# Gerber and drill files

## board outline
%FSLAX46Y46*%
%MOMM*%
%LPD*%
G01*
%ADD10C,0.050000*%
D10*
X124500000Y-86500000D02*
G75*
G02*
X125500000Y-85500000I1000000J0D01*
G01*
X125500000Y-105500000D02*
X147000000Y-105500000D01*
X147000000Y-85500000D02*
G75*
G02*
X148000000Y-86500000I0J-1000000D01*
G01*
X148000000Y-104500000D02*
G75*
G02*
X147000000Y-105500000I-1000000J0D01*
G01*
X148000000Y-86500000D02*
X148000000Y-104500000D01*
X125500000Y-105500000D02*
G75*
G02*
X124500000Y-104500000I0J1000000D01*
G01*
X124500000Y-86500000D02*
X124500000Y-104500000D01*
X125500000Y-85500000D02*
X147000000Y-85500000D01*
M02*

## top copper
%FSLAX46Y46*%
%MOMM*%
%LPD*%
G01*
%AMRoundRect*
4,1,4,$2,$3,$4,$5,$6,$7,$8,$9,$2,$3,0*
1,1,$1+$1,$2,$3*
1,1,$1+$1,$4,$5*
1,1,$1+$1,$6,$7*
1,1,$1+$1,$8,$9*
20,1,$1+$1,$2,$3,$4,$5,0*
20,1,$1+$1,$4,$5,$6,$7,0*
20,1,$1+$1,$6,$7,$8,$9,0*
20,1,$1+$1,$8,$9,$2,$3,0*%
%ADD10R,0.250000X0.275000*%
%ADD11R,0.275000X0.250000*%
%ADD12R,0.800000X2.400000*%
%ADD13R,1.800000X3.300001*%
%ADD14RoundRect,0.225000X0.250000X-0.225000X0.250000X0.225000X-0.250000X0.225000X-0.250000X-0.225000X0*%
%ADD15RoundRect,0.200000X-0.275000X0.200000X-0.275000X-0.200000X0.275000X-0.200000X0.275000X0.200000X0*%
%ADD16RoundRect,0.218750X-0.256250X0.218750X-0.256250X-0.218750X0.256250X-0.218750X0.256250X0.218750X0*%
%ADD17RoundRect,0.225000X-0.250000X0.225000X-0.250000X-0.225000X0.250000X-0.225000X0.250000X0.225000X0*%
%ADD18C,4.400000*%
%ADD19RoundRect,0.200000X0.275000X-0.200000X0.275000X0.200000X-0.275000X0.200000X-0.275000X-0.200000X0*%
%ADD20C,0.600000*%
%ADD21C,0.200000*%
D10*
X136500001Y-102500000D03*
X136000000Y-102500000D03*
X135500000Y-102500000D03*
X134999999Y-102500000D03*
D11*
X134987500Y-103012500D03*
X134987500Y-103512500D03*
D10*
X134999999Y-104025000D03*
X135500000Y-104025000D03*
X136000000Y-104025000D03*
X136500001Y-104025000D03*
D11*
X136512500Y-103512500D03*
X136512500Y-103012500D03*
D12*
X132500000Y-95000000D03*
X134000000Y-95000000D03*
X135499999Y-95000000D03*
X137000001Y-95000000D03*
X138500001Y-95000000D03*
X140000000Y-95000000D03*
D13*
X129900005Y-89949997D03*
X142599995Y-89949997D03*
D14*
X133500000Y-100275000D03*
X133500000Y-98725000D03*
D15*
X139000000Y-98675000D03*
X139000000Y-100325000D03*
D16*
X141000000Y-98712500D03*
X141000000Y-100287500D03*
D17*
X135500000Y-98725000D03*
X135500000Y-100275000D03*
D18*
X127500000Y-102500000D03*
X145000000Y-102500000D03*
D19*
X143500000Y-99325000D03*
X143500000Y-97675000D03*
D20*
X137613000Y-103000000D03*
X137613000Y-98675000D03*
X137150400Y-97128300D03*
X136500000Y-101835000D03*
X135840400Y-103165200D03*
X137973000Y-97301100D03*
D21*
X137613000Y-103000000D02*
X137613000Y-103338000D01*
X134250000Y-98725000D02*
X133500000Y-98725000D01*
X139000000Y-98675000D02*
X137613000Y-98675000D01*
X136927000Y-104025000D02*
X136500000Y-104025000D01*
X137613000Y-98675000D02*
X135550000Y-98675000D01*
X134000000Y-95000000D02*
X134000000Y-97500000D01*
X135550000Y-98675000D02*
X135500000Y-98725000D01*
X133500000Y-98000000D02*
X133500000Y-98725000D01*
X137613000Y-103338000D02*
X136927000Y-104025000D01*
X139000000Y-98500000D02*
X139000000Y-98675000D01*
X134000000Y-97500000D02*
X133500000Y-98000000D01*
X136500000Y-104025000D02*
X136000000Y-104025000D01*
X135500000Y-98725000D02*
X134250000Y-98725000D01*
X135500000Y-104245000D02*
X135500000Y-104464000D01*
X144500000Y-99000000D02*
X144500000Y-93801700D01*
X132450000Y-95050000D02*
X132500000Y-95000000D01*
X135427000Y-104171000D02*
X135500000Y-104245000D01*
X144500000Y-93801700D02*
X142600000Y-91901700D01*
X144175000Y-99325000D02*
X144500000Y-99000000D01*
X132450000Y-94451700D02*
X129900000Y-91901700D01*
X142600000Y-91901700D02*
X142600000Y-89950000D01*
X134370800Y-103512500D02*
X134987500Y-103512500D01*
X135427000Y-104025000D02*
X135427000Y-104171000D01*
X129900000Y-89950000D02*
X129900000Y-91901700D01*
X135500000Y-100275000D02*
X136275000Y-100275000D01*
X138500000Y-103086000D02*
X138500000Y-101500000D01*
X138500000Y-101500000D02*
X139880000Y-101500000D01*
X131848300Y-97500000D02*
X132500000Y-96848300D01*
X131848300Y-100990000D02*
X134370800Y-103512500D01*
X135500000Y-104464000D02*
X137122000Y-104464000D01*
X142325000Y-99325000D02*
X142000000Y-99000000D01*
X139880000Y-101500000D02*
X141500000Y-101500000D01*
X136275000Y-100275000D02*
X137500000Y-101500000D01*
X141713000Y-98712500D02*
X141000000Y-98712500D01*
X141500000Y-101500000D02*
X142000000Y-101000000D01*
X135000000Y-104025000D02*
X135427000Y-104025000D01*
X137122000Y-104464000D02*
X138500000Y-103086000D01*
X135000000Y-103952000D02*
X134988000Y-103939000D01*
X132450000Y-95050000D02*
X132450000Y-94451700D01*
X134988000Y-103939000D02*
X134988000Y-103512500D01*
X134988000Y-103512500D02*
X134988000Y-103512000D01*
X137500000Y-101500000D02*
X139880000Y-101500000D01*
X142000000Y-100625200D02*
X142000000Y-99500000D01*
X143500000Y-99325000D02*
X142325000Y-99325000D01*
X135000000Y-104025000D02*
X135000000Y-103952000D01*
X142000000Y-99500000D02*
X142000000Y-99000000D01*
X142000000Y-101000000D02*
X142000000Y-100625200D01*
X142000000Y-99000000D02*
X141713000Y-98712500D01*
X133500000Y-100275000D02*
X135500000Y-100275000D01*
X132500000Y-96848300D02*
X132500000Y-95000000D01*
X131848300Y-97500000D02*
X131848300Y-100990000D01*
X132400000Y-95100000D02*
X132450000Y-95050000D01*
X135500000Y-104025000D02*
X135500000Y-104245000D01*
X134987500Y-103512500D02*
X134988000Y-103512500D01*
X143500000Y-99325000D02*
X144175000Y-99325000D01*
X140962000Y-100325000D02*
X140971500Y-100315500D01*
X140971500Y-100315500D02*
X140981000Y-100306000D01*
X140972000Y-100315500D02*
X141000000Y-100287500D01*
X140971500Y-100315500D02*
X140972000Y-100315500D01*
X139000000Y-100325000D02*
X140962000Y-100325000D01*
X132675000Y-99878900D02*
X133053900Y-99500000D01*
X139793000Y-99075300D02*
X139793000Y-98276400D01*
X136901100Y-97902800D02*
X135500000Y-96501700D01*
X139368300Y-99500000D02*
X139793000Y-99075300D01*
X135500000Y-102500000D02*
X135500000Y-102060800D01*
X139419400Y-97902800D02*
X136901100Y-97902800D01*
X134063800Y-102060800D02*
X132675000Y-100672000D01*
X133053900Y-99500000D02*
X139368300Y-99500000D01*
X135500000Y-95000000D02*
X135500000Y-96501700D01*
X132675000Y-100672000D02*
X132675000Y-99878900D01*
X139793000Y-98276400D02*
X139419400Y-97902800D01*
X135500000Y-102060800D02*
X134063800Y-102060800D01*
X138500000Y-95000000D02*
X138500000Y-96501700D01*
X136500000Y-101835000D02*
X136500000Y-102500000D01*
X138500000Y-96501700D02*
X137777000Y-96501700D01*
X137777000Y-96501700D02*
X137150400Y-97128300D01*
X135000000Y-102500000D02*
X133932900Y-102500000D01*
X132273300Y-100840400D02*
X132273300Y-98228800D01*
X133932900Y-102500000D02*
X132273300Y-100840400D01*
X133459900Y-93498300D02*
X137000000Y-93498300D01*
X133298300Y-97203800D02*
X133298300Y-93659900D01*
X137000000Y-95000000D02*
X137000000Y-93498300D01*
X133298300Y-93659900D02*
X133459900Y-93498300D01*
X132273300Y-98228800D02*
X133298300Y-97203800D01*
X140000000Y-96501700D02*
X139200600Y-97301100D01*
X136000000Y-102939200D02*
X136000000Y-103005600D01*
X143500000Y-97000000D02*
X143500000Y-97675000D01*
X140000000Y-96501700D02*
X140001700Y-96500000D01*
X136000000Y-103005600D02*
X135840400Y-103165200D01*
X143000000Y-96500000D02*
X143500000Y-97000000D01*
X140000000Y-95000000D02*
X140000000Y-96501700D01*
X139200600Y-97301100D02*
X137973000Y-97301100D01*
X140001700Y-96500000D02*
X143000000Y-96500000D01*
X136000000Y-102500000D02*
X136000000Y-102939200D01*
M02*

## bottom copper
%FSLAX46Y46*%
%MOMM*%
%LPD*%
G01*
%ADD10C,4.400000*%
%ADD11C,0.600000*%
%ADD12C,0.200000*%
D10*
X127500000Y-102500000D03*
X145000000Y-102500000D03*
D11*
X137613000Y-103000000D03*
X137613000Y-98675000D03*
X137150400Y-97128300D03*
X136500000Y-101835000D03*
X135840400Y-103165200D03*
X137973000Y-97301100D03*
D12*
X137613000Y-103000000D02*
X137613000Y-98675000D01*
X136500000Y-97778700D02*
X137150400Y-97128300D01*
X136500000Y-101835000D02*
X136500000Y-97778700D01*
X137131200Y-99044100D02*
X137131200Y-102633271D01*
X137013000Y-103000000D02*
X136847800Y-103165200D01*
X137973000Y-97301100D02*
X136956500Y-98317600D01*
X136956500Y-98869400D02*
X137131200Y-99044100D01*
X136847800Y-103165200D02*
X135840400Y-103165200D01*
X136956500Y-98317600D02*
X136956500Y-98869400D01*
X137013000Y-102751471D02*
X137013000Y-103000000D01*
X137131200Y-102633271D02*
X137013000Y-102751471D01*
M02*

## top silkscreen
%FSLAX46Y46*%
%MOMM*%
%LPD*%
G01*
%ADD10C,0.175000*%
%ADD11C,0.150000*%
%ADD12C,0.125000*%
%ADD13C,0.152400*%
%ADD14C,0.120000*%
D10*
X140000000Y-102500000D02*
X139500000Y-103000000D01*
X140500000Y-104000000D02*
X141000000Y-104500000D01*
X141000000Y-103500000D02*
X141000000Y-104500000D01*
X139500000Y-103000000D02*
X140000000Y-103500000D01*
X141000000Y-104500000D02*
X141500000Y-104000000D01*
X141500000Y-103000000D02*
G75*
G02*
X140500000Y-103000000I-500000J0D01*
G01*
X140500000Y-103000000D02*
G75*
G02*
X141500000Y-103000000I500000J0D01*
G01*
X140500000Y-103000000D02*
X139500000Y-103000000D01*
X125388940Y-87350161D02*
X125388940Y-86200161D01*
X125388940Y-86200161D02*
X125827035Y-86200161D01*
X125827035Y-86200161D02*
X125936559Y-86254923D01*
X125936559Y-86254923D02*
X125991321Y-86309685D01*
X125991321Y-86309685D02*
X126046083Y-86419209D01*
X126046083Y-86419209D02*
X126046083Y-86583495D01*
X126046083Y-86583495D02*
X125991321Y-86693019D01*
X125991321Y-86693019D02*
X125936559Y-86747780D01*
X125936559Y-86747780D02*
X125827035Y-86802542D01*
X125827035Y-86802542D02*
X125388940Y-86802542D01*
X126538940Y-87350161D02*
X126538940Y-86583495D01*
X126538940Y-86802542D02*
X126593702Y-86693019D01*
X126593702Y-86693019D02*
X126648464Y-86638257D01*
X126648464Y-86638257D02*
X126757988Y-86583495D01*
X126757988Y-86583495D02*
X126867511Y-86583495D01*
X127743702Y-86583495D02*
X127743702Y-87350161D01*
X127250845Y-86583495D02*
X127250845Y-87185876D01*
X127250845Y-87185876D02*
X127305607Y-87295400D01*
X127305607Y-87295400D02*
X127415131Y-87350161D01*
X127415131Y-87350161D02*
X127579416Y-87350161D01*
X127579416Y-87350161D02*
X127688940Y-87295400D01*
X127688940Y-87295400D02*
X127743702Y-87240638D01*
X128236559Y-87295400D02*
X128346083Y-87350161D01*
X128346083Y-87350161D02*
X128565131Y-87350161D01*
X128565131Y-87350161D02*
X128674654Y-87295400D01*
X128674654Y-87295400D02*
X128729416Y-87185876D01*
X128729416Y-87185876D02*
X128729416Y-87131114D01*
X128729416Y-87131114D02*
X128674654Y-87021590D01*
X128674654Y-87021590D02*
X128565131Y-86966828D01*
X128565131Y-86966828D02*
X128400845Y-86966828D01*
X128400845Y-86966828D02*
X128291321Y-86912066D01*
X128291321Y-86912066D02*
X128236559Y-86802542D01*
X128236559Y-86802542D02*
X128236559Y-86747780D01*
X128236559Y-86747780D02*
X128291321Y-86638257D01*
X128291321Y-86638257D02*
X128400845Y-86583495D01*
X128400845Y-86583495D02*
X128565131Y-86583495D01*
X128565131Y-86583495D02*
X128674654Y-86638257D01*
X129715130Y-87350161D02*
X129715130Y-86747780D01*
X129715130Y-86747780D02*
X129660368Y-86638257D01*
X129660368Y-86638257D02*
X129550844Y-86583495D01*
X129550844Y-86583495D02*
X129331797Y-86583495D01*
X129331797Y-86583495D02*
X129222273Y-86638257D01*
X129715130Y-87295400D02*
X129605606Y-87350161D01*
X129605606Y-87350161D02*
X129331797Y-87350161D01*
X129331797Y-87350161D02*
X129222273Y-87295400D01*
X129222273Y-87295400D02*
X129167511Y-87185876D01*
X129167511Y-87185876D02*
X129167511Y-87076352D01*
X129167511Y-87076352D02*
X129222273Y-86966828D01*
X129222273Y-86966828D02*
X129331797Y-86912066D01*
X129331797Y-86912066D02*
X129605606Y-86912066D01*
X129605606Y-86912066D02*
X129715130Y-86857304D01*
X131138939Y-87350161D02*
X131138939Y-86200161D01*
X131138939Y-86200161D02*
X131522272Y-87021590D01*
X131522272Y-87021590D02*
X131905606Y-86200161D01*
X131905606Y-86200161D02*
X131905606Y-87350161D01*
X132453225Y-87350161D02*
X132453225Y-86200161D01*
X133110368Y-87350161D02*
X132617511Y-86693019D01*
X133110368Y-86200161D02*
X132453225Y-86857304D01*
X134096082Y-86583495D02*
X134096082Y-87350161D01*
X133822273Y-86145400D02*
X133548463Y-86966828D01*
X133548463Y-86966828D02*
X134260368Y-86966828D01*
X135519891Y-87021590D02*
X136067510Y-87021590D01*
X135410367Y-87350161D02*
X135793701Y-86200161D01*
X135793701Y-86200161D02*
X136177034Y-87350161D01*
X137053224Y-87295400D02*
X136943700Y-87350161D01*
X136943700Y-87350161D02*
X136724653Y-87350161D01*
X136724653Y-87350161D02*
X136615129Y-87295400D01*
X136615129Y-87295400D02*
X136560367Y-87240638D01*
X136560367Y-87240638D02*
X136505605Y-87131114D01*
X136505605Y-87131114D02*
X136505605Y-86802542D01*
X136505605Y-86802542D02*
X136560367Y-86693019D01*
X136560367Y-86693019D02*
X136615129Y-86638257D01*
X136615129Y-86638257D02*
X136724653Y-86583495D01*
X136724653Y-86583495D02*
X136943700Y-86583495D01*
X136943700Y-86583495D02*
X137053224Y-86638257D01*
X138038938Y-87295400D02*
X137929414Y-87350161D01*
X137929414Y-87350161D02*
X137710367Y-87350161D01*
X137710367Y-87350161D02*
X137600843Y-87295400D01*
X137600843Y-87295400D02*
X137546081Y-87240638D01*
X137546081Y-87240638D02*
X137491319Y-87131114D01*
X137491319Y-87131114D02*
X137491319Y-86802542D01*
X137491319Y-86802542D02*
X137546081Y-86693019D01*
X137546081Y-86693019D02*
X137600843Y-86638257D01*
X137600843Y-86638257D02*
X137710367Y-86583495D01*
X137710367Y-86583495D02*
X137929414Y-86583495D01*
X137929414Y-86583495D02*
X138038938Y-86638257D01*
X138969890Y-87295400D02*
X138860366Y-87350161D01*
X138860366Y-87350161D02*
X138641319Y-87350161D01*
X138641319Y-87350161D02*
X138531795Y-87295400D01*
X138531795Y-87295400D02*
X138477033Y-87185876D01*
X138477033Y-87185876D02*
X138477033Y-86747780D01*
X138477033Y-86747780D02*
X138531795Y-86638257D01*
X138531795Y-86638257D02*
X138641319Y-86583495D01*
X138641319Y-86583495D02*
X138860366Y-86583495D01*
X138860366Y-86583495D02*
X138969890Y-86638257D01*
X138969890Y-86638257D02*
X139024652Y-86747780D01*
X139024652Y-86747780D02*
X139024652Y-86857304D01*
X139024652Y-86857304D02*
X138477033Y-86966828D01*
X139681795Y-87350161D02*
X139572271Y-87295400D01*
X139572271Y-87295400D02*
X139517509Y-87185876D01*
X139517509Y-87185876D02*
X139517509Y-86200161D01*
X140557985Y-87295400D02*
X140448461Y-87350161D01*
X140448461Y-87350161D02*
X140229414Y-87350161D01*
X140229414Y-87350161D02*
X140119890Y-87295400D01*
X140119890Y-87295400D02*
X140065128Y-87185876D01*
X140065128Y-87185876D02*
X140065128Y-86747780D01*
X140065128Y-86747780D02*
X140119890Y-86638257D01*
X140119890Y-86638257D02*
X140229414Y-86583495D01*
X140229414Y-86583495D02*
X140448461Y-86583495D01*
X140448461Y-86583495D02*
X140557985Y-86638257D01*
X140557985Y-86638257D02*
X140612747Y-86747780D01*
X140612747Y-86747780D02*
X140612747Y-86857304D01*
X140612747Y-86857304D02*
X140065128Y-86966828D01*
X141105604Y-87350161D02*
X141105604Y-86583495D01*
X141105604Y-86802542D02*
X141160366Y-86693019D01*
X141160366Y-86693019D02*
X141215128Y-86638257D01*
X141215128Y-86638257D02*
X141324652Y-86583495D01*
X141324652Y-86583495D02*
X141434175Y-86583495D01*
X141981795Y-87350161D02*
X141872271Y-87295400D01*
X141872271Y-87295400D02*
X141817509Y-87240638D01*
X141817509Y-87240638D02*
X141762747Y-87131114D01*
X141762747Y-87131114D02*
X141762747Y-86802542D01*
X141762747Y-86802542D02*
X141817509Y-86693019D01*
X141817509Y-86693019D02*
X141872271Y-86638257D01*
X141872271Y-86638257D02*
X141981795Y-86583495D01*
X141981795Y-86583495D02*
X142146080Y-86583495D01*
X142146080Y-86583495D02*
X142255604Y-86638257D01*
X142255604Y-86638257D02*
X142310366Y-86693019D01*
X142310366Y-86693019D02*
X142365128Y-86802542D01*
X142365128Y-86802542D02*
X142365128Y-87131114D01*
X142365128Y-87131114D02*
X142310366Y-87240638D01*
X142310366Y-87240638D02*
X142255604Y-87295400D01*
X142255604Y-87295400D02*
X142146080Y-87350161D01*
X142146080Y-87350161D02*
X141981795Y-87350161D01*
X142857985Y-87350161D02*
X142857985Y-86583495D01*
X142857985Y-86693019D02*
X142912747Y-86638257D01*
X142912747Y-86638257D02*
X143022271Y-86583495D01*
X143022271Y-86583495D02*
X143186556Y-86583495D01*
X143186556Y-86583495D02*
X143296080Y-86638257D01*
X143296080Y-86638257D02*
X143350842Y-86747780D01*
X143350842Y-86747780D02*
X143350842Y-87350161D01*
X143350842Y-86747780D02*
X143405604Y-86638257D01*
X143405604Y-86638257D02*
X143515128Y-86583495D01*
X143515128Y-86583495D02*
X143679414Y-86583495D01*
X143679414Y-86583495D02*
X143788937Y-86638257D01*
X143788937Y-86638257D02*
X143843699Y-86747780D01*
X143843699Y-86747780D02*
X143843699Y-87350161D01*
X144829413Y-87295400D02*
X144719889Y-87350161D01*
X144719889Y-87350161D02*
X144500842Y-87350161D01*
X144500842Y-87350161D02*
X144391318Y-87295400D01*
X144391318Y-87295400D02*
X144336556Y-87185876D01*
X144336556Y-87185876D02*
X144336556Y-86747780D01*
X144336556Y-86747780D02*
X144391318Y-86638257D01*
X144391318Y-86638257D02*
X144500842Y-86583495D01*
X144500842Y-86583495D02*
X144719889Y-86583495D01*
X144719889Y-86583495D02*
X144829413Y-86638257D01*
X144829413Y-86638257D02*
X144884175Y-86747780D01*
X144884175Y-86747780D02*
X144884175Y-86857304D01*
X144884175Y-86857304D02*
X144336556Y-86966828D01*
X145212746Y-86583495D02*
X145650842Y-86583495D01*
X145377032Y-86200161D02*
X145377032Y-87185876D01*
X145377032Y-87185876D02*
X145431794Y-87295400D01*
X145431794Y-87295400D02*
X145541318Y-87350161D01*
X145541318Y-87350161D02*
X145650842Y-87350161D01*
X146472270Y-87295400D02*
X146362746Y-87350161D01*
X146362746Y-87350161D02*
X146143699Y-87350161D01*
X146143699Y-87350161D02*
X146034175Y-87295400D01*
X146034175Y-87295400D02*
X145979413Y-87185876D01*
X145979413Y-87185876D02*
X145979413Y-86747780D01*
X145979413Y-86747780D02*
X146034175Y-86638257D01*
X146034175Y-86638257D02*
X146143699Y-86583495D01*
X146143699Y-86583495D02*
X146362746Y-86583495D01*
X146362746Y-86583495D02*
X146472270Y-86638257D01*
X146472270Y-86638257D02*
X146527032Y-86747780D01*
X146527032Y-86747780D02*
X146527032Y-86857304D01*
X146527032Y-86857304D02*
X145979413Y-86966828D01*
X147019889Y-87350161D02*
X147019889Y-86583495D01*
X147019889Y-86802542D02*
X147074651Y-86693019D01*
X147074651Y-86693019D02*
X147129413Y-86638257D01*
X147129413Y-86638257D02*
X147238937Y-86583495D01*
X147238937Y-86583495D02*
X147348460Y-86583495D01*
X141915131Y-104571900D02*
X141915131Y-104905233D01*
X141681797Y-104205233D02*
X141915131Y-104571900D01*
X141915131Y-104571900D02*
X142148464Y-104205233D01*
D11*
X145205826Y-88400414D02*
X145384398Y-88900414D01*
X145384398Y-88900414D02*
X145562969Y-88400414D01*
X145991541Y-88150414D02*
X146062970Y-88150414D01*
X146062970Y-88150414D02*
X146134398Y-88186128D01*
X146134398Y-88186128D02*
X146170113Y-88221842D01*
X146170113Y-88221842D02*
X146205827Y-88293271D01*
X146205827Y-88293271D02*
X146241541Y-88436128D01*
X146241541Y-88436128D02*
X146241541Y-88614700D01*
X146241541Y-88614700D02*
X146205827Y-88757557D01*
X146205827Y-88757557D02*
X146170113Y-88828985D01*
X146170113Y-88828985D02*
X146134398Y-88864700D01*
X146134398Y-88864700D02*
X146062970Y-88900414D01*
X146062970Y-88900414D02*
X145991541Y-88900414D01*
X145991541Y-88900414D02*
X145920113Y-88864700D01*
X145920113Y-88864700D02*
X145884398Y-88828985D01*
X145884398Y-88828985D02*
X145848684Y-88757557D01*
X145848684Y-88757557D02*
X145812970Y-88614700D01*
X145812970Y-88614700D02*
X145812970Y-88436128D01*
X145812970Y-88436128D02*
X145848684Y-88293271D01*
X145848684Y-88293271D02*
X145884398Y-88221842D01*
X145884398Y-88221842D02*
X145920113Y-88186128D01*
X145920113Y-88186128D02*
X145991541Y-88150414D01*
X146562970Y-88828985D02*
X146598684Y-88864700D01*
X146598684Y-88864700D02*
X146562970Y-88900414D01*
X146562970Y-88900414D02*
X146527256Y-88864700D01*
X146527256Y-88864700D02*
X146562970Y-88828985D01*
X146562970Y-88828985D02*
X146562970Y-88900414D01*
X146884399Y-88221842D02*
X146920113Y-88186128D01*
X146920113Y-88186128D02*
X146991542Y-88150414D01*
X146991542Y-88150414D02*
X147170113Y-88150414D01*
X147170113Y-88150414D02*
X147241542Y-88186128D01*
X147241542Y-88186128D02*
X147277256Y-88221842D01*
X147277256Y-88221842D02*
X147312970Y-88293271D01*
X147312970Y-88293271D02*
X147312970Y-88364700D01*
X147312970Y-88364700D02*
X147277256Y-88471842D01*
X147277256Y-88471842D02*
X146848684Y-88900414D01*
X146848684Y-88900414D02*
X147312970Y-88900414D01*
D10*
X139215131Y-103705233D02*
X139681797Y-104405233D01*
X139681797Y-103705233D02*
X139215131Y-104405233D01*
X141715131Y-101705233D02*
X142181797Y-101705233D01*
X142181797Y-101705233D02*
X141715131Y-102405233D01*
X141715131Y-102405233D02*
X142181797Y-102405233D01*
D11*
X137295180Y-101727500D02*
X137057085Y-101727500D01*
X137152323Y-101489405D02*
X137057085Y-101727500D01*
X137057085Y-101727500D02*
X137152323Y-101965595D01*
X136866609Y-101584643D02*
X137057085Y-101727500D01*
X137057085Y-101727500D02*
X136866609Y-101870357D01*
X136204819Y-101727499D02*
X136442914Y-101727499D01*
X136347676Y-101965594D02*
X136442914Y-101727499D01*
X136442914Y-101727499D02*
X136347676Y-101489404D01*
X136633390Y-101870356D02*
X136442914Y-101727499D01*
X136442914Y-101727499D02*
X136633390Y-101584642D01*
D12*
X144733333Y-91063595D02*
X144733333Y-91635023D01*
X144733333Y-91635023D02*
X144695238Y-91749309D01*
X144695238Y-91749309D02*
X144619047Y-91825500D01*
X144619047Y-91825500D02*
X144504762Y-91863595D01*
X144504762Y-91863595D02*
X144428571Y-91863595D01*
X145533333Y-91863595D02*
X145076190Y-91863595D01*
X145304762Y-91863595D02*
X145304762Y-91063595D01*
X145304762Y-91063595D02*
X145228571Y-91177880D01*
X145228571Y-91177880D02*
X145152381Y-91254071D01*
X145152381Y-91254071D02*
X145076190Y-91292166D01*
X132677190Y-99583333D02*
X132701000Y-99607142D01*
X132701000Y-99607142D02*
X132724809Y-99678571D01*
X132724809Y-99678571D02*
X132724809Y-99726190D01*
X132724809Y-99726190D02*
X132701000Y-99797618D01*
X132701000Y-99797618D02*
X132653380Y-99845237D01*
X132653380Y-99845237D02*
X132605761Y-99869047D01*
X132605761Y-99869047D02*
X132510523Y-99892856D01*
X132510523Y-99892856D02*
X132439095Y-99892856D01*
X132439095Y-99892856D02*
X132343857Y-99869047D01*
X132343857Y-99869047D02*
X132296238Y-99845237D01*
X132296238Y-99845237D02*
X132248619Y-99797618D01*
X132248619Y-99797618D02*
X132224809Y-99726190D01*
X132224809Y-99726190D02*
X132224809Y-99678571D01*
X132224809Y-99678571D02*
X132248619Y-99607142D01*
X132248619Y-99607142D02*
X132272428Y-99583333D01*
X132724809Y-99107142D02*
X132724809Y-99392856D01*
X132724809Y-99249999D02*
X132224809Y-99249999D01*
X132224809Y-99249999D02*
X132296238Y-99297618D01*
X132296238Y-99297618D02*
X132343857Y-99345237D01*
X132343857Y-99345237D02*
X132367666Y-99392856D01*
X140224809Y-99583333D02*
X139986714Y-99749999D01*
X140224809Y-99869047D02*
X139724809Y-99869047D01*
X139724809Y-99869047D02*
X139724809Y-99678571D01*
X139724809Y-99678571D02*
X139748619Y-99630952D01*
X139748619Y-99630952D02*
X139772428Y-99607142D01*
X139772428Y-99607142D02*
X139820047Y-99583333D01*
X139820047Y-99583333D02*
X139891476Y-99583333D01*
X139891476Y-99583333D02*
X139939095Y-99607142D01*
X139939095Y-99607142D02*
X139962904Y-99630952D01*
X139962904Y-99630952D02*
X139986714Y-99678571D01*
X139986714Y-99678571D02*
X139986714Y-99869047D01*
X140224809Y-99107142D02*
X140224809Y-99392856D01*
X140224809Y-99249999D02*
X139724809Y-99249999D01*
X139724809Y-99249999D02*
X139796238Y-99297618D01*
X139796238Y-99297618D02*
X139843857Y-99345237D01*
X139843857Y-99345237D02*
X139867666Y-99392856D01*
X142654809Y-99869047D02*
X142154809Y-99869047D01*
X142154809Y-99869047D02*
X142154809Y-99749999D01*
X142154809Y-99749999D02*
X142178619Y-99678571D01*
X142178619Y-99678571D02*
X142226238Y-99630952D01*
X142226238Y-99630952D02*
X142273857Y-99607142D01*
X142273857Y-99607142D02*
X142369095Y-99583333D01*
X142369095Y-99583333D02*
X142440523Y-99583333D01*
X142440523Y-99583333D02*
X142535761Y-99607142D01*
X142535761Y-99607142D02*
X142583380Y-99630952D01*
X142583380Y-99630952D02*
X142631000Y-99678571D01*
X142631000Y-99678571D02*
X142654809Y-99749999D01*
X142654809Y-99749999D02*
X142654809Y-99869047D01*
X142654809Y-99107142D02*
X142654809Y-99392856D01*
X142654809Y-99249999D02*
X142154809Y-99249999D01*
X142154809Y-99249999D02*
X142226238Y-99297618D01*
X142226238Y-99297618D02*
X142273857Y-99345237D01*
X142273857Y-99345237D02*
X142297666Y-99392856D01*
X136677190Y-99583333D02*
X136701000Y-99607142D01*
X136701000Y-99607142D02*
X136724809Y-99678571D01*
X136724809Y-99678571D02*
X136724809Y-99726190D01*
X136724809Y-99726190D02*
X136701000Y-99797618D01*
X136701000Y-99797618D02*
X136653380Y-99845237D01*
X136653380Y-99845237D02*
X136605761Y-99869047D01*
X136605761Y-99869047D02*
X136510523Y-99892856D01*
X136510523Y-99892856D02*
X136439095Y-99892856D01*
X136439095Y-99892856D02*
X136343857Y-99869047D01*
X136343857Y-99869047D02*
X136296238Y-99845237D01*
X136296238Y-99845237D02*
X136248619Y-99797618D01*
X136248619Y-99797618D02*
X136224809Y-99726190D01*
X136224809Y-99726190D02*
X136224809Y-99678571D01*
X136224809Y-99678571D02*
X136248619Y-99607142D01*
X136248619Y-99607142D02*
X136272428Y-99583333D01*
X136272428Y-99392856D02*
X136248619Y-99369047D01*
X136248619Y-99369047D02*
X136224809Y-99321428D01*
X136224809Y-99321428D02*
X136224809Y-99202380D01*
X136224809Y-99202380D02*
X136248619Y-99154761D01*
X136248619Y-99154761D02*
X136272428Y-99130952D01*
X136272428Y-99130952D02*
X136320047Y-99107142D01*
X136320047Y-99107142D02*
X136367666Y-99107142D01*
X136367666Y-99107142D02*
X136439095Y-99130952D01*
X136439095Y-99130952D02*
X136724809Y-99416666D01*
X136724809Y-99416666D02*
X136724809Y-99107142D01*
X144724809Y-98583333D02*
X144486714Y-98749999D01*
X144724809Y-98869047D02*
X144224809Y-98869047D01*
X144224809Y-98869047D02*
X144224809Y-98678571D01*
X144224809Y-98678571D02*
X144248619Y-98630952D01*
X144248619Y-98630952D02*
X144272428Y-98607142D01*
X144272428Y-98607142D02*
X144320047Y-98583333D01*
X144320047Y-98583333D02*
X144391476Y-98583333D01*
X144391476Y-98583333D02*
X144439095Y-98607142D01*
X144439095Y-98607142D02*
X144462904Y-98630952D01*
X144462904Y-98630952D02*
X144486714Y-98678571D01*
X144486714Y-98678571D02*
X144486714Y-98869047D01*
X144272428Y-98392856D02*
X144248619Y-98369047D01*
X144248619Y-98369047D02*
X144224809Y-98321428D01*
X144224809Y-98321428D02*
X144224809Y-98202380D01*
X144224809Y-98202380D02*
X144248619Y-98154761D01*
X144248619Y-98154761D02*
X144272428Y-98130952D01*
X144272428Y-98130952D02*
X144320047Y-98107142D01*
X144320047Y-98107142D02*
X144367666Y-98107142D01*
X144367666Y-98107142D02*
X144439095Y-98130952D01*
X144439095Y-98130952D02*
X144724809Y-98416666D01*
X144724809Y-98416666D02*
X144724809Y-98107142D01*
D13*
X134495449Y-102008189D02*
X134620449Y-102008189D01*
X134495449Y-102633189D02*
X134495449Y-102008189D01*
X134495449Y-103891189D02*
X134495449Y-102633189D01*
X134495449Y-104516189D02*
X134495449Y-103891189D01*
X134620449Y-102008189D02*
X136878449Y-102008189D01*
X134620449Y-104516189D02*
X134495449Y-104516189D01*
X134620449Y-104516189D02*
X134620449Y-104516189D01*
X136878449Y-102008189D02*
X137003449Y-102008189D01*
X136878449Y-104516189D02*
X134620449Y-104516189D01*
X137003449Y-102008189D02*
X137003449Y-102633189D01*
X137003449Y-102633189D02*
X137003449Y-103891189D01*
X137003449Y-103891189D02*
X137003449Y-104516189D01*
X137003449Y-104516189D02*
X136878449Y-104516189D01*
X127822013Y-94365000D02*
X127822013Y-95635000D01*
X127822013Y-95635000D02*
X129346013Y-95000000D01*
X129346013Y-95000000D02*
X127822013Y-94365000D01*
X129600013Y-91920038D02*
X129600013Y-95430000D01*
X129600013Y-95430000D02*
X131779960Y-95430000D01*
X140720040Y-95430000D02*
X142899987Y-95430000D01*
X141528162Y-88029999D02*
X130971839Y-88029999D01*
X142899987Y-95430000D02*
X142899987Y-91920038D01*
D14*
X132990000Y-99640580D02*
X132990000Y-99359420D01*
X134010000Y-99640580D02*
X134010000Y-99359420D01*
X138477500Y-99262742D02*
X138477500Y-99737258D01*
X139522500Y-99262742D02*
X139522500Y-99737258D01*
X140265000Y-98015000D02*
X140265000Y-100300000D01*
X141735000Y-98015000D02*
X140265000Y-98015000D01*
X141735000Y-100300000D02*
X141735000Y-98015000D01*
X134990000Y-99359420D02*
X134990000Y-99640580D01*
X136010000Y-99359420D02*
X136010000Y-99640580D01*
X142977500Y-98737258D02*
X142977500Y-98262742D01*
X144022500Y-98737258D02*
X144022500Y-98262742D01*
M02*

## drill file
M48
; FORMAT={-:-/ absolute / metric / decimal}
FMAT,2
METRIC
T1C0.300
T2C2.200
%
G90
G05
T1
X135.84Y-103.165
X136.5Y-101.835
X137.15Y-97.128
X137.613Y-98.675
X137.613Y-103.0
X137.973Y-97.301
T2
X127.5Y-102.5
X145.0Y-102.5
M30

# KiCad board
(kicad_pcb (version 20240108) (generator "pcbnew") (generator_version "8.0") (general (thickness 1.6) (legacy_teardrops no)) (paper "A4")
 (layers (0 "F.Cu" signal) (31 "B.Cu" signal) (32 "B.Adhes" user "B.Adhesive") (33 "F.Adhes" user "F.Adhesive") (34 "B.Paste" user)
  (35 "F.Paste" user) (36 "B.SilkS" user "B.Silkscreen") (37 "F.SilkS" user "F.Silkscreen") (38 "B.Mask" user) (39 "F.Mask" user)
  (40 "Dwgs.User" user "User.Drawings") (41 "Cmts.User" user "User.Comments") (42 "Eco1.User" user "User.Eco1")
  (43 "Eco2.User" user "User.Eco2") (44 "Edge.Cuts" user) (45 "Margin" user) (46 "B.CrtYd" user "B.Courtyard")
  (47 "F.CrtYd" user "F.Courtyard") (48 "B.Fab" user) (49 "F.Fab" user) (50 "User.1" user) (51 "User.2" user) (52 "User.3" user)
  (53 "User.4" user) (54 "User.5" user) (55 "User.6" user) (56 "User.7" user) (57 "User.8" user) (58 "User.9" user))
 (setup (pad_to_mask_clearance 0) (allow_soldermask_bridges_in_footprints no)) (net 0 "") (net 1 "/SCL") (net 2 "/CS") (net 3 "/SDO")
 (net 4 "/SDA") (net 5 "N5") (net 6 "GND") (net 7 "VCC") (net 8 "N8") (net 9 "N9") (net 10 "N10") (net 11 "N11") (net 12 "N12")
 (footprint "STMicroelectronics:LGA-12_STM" (layer "F.Cu") (at 135.75 103.2625 -90)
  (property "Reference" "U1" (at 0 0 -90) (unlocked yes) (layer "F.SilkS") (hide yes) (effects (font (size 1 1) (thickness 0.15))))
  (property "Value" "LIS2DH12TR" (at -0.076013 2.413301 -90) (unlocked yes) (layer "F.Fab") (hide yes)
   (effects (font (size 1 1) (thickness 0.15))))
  (fp_line (start -1.254311 1.254551) (end -1.254311 1.129551) (stroke (width 0.1524) (type solid)) (layer "F.SilkS"))
  (fp_line (start -0.629311 1.254551) (end -1.254311 1.254551) (stroke (width 0.1524) (type solid)) (layer "F.SilkS"))
  (fp_line (start 0.628689 1.254551) (end -0.629311 1.254551) (stroke (width 0.1524) (type solid)) (layer "F.SilkS"))
  (fp_line (start 1.253689 1.254551) (end 0.628689 1.254551) (stroke (width 0.1524) (type solid)) (layer "F.SilkS"))
  (fp_line (start -1.254311 1.129551) (end -1.254311 -1.128449) (stroke (width 0.1524) (type solid)) (layer "F.SilkS"))
  (fp_line (start 1.253689 1.129551) (end 1.253689 1.254551) (stroke (width 0.1524) (type solid)) (layer "F.SilkS"))
  (fp_line (start 1.253689 1.129551) (end 1.253689 1.129551) (stroke (width 0.1524) (type solid)) (layer "F.SilkS"))
  (fp_line (start -1.254311 -1.128449) (end -1.254311 -1.253449) (stroke (width 0.1524) (type solid)) (layer "F.SilkS"))
  (fp_line (start 1.253689 -1.128449) (end 1.253689 1.129551) (stroke (width 0.1524) (type solid)) (layer "F.SilkS"))
  (fp_line (start -1.254311 -1.253449) (end -0.629311 -1.253449) (stroke (width 0.1524) (type solid)) (layer "F.SilkS"))
  (fp_line (start -0.629311 -1.253449) (end 0.628689 -1.253449) (stroke (width 0.1524) (type solid)) (layer "F.SilkS"))
  (fp_line (start 0.628689 -1.253449) (end 1.253689 -1.253449) (stroke (width 0.1524) (type solid)) (layer "F.SilkS"))
  (fp_line (start 1.253689 -1.253449) (end 1.253689 -1.128449) (stroke (width 0.1524) (type solid)) (layer "F.SilkS"))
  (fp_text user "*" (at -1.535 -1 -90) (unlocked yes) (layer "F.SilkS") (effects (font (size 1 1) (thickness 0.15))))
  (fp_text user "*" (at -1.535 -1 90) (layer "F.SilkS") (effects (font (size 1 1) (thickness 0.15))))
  (pad "1" smd rect (at -0.7625 -0.750001) (size 0.25 0.275) (layers "F.Cu" "F.Paste" "F.Mask") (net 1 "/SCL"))
  (pad "2" smd rect (at -0.7625 -0.25) (size 0.25 0.275) (layers "F.Cu" "F.Paste" "F.Mask") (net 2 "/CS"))
  (pad "3" smd rect (at -0.7625 0.25) (size 0.25 0.275) (layers "F.Cu" "F.Paste" "F.Mask") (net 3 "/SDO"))
  (pad "4" smd rect (at -0.7625 0.750001) (size 0.25 0.275) (layers "F.Cu" "F.Paste" "F.Mask") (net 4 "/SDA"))
  (pad "5" smd rect (at -0.25 0.7625 270) (size 0.25 0.275) (layers "F.Cu" "F.Paste" "F.Mask") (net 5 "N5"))
  (pad "6" smd rect (at 0.25 0.7625 270) (size 0.25 0.275) (layers "F.Cu" "F.Paste" "F.Mask") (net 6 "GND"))
  (pad "7" smd rect (at 0.7625 0.750001) (size 0.25 0.275) (layers "F.Cu" "F.Paste" "F.Mask") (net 6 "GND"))
  (pad "8" smd rect (at 0.7625 0.25) (size 0.25 0.275) (layers "F.Cu" "F.Paste" "F.Mask") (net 6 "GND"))
  (pad "9" smd rect (at 0.7625 -0.25) (size 0.25 0.275) (layers "F.Cu" "F.Paste" "F.Mask") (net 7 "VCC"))
  (pad "10" smd rect (at 0.7625 -0.750001) (size 0.25 0.275) (layers "F.Cu" "F.Paste" "F.Mask") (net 7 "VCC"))
  (pad "11" smd rect (at 0.25 -0.7625 270) (size 0.25 0.275) (layers "F.Cu" "F.Paste" "F.Mask") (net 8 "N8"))
  (pad "12" smd rect (at -0.25 -0.7625 270) (size 0.25 0.275) (layers "F.Cu" "F.Paste" "F.Mask") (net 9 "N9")))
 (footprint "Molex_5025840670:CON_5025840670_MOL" (layer "F.Cu") (at 132.5 95)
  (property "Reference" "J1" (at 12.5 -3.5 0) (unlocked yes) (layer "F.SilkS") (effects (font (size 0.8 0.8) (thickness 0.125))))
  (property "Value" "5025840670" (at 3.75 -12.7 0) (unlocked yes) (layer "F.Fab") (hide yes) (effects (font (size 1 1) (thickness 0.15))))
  (fp_line (start -4.677987 -0.635) (end -4.677987 0.635) (stroke (width 0.1524) (type solid)) (layer "F.SilkS"))
  (fp_line (start -4.677987 0.635) (end -3.153987 0) (stroke (width 0.1524) (type solid)) (layer "F.SilkS"))
  (fp_line (start -3.153987 0) (end -4.677987 -0.635) (stroke (width 0.1524) (type solid)) (layer "F.SilkS"))
  (fp_line (start -2.899987 -3.079962) (end -2.899987 0.43) (stroke (width 0.1524) (type solid)) (layer "F.SilkS"))
  (fp_line (start -2.899987 0.43) (end -0.72004 0.43) (stroke (width 0.1524) (type solid)) (layer "F.SilkS"))
  (fp_line (start 8.22004 0.43) (end 10.399987 0.43) (stroke (width 0.1524) (type solid)) (layer "F.SilkS"))
  (fp_line (start 9.028162 -6.970001) (end -1.528161 -6.970001) (stroke (width 0.1524) (type solid)) (layer "F.SilkS"))
  (fp_line (start 10.399987 0.43) (end 10.399987 -3.079962) (stroke (width 0.1524) (type solid)) (layer "F.SilkS"))
  (pad "1" smd rect (at 0 0) (size 0.8 2.4) (layers "F.Cu" "F.Paste" "F.Mask") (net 6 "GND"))
  (pad "2" smd rect (at 1.5 0) (size 0.8 2.4) (layers "F.Cu" "F.Paste" "F.Mask") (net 7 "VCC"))
  (pad "3" smd rect (at 2.999999 0) (size 0.8 2.4) (layers "F.Cu" "F.Paste" "F.Mask") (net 3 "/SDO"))
  (pad "4" smd rect (at 4.500001 0) (size 0.8 2.4) (layers "F.Cu" "F.Paste" "F.Mask") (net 4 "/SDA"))
  (pad "5" smd rect (at 6.000001 0) (size 0.8 2.4) (layers "F.Cu" "F.Paste" "F.Mask") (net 1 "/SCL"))
  (pad "6" smd rect (at 7.5 0) (size 0.8 2.4) (layers "F.Cu" "F.Paste" "F.Mask") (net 2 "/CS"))
  (pad "7" smd rect (at -2.599995 -5.050003) (size 1.8 3.300001) (layers "F.Cu" "F.Paste" "F.Mask") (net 6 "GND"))
  (pad "8" smd rect (at 10.099995 -5.050003) (size 1.8 3.300001) (layers "F.Cu" "F.Paste" "F.Mask") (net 6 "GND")))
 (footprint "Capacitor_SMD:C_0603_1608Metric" (layer "F.Cu") (at 133.5 99.5 90)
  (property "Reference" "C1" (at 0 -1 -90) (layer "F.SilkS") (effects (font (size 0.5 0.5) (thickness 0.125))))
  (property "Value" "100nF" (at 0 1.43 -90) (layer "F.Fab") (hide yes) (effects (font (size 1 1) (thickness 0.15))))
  (fp_line (start -0.14058 -0.51) (end 0.14058 -0.51) (stroke (width 0.12) (type solid)) (layer "F.SilkS"))
  (fp_line (start -0.14058 0.51) (end 0.14058 0.51) (stroke (width 0.12) (type solid)) (layer "F.SilkS"))
  (pad "1" smd roundrect (at -0.775 0 90) (size 0.9 0.95) (layers "F.Cu" "F.Paste" "F.Mask") (roundrect_rratio 0.25) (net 6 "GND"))
  (pad "2" smd roundrect (at 0.775 0 90) (size 0.9 0.95) (layers "F.Cu" "F.Paste" "F.Mask") (roundrect_rratio 0.25) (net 7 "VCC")))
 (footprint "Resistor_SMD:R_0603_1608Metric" (layer "F.Cu") (at 139 99.5 -90)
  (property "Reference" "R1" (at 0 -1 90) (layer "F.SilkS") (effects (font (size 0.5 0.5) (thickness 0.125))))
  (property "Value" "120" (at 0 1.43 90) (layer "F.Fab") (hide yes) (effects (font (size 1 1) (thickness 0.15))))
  (fp_line (start -0.237258 0.5225) (end 0.237258 0.5225) (stroke (width 0.12) (type solid)) (layer "F.SilkS"))
  (fp_line (start -0.237258 -0.5225) (end 0.237258 -0.5225) (stroke (width 0.12) (type solid)) (layer "F.SilkS"))
  (pad "1" smd roundrect (at -0.825 0 270) (size 0.8 0.95) (layers "F.Cu" "F.Paste" "F.Mask") (roundrect_rratio 0.25) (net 7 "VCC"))
  (pad "2" smd roundrect (at 0.825 0 270) (size 0.8 0.95) (layers "F.Cu" "F.Paste" "F.Mask") (roundrect_rratio 0.25) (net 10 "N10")))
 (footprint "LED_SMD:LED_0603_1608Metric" (layer "F.Cu") (at 141 99.5 -90)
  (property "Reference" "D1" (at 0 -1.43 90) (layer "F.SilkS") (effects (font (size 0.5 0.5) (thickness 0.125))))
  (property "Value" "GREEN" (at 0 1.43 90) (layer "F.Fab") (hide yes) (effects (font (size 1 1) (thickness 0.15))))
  (fp_line (start -1.485 0.735) (end 0.8 0.735) (stroke (width 0.12) (type solid)) (layer "F.SilkS"))
  (fp_line (start -1.485 -0.735) (end -1.485 0.735) (stroke (width 0.12) (type solid)) (layer "F.SilkS"))
  (fp_line (start 0.8 -0.735) (end -1.485 -0.735) (stroke (width 0.12) (type solid)) (layer "F.SilkS"))
  (pad "1" smd roundrect (at -0.7875 0 270) (size 0.875 0.95) (layers "F.Cu" "F.Paste" "F.Mask") (roundrect_rratio 0.25) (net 6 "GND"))
  (pad "2" smd roundrect (at 0.7875 0 270) (size 0.875 0.95) (layers "F.Cu" "F.Paste" "F.Mask") (roundrect_rratio 0.25) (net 10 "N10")))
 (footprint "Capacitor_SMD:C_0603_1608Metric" (layer "F.Cu") (at 135.5 99.5 -90)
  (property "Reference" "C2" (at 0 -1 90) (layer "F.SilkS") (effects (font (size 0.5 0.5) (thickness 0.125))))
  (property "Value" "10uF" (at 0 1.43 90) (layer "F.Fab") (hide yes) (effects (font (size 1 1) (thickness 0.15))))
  (fp_line (start -0.14058 0.51) (end 0.14058 0.51) (stroke (width 0.12) (type solid)) (layer "F.SilkS"))
  (fp_line (start -0.14058 -0.51) (end 0.14058 -0.51) (stroke (width 0.12) (type solid)) (layer "F.SilkS"))
  (pad "1" smd roundrect (at -0.775 0 270) (size 0.9 0.95) (layers "F.Cu" "F.Paste" "F.Mask") (roundrect_rratio 0.25) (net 7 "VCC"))
  (pad "2" smd roundrect (at 0.775 0 270) (size 0.9 0.95) (layers "F.Cu" "F.Paste" "F.Mask") (roundrect_rratio 0.25) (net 6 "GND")))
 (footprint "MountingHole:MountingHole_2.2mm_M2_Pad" (layer "F.Cu") (at 127.5 102.5)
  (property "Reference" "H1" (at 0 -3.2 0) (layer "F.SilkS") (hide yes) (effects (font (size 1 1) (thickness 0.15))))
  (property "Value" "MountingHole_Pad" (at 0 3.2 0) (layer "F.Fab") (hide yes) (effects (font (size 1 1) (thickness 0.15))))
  (pad "1" thru_hole circle (at 0 0) (size 4.4 4.4) (drill 2.2) (layers "*.Cu" "*.Mask") (remove_unused_layers no) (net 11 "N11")))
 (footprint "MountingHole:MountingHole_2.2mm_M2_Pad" (layer "F.Cu") (at 145 102.5)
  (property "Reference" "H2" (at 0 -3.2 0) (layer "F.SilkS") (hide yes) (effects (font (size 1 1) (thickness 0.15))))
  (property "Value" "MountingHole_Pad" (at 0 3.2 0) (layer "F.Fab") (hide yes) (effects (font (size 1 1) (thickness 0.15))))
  (pad "1" thru_hole circle (at 0 0) (size 4.4 4.4) (drill 2.2) (layers "*.Cu" "*.Mask") (remove_unused_layers no) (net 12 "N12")))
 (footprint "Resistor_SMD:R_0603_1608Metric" (layer "F.Cu") (at 143.5 98.5 90)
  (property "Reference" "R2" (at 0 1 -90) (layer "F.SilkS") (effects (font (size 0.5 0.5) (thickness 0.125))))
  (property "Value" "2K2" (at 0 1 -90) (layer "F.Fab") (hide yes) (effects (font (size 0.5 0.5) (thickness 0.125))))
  (fp_line (start -0.237258 -0.5225) (end 0.237258 -0.5225) (stroke (width 0.12) (type solid)) (layer "F.SilkS"))
  (fp_line (start -0.237258 0.5225) (end 0.237258 0.5225) (stroke (width 0.12) (type solid)) (layer "F.SilkS"))
  (pad "1" smd roundrect (at -0.825 0 90) (size 0.8 0.95) (layers "F.Cu" "F.Paste" "F.Mask") (roundrect_rratio 0.25) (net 6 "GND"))
  (pad "2" smd roundrect (at 0.825 0 90) (size 0.8 0.95) (layers "F.Cu" "F.Paste" "F.Mask") (roundrect_rratio 0.25) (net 2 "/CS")))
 (gr_line (start 140 102.5) (end 139.5 103) (stroke (width 0.175) (type default)) (layer "F.SilkS"))
 (gr_line (start 140.5 104) (end 141 104.5) (stroke (width 0.175) (type default)) (layer "F.SilkS"))
 (gr_line (start 141 103.5) (end 141 104.5) (stroke (width 0.175) (type default)) (layer "F.SilkS"))
 (gr_line (start 139.5 103) (end 140 103.5) (stroke (width 0.175) (type default)) (layer "F.SilkS"))
 (gr_line (start 141 104.5) (end 141.5 104) (stroke (width 0.175) (type default)) (layer "F.SilkS"))
 (gr_circle (center 141 103) (end 141.5 103) (stroke (width 0.175) (type default)) (fill none) (layer "F.SilkS"))
 (gr_line (start 140.5 103) (end 139.5 103) (stroke (width 0.175) (type default)) (layer "F.SilkS"))
 (gr_arc (start 124.5 86.5) (mid 124.792893 85.792893) (end 125.5 85.5) (stroke (width 0.05) (type default)) (layer "Edge.Cuts"))
 (gr_line (start 125.5 105.5) (end 147 105.5) (stroke (width 0.05) (type default)) (layer "Edge.Cuts"))
 (gr_arc (start 147 85.5) (mid 147.707107 85.792893) (end 148 86.5) (stroke (width 0.05) (type default)) (layer "Edge.Cuts"))
 (gr_arc (start 148 104.5) (mid 147.707107 105.207107) (end 147 105.5) (stroke (width 0.05) (type default)) (layer "Edge.Cuts"))
 (gr_line (start 148 86.5) (end 148 104.5) (stroke (width 0.05) (type default)) (layer "Edge.Cuts"))
 (gr_arc (start 125.5 105.5) (mid 124.792893 105.207107) (end 124.5 104.5) (stroke (width 0.05) (type default)) (layer "Edge.Cuts"))
 (gr_line (start 124.5 86.5) (end 124.5 104.5) (stroke (width 0.05) (type default)) (layer "Edge.Cuts"))
 (gr_line (start 125.5 85.5) (end 147 85.5) (stroke (width 0.05) (type default)) (layer "Edge.Cuts"))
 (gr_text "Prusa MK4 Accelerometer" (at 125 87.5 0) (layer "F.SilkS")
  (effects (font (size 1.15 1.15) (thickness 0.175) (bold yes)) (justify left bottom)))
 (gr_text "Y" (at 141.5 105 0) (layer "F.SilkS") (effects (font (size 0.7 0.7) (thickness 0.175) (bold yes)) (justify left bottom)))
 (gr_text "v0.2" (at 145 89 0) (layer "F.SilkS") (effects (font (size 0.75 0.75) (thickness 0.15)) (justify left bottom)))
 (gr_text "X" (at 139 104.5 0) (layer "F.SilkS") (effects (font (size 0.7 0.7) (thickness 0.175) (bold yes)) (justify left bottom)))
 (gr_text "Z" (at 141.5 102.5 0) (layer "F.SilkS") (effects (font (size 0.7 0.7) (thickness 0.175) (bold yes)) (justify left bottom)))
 (segment (start 137.613 103) (end 137.613 103.338) (width 0.2) (layer "F.Cu") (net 7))
 (segment (start 134.25 98.725) (end 133.5 98.725) (width 0.2) (layer "F.Cu") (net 7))
 (segment (start 139 98.675) (end 137.613 98.675) (width 0.2) (layer "F.Cu") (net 7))
 (segment (start 136.927 104.025) (end 136.5 104.025) (width 0.2) (layer "F.Cu") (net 7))
 (segment (start 137.613 98.675) (end 135.55 98.675) (width 0.2) (layer "F.Cu") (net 7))
 (segment (start 134 95) (end 134 97.5) (width 0.2) (layer "F.Cu") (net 7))
 (segment (start 135.55 98.675) (end 135.5 98.725) (width 0.2) (layer "F.Cu") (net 7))
 (segment (start 133.5 98) (end 133.5 98.725) (width 0.2) (layer "F.Cu") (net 7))
 (segment (start 137.613 103.338) (end 136.927 104.025) (width 0.2) (layer "F.Cu") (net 7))
 (segment (start 139 98.5) (end 139 98.675) (width 0.2) (layer "F.Cu") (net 7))
 (segment (start 134 97.5) (end 133.5 98) (width 0.2) (layer "F.Cu") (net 7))
 (segment (start 136.5 104.025) (end 136 104.025) (width 0.2) (layer "F.Cu") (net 7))
 (segment (start 135.5 98.725) (end 134.25 98.725) (width 0.2) (layer "F.Cu") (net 7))
 (via (at 137.613 103) (size 0.6) (drill 0.3) (layers "F.Cu" "B.Cu") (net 7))
 (via (at 137.613 98.675) (size 0.6) (drill 0.3) (layers "F.Cu" "B.Cu") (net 7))
 (segment (start 137.613 103) (end 137.613 98.675) (width 0.2) (layer "B.Cu") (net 7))
 (segment (start 135.5 104.245) (end 135.5 104.464) (width 0.2) (layer "F.Cu") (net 6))
 (segment (start 144.5 99) (end 144.5 93.8017) (width 0.2) (layer "F.Cu") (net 6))
 (segment (start 132.45 95.05) (end 132.5 95) (width 0.2) (layer "F.Cu") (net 6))
 (segment (start 135.427 104.171) (end 135.5 104.245) (width 0.2) (layer "F.Cu") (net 6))
 (segment (start 144.5 93.8017) (end 142.6 91.9017) (width 0.2) (layer "F.Cu") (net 6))
 (segment (start 144.175 99.325) (end 144.5 99) (width 0.2) (layer "F.Cu") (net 6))
 (segment (start 132.45 94.4517) (end 129.9 91.9017) (width 0.2) (layer "F.Cu") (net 6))
 (segment (start 142.6 91.9017) (end 142.6 89.95) (width 0.2) (layer "F.Cu") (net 6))
 (segment (start 134.3708 103.5125) (end 134.9875 103.5125) (width 0.2) (layer "F.Cu") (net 6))
 (segment (start 135.427 104.025) (end 135.427 104.171) (width 0.2) (layer "F.Cu") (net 6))
 (segment (start 129.9 89.95) (end 129.9 91.9017) (width 0.2) (layer "F.Cu") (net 6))
 (segment (start 135.5 100.275) (end 136.275 100.275) (width 0.2) (layer "F.Cu") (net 6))
 (segment (start 138.5 103.086) (end 138.5 101.5) (width 0.2) (layer "F.Cu") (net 6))
 (segment (start 138.5 101.5) (end 139.88 101.5) (width 0.2) (layer "F.Cu") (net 6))
 (segment (start 131.8483 97.5) (end 132.5 96.8483) (width 0.2) (layer "F.Cu") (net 6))
 (segment (start 131.8483 100.99) (end 134.3708 103.5125) (width 0.2) (layer "F.Cu") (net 6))
 (segment (start 135.5 104.464) (end 137.122 104.464) (width 0.2) (layer "F.Cu") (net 6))
 (segment (start 142.325 99.325) (end 142 99) (width 0.2) (layer "F.Cu") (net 6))
 (segment (start 139.88 101.5) (end 141.5 101.5) (width 0.2) (layer "F.Cu") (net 6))
 (segment (start 136.275 100.275) (end 137.5 101.5) (width 0.2) (layer "F.Cu") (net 6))
 (segment (start 141.713 98.7125) (end 141 98.7125) (width 0.2) (layer "F.Cu") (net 6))
 (segment (start 141.5 101.5) (end 142 101) (width 0.2) (layer "F.Cu") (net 6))
 (segment (start 135 104.025) (end 135.427 104.025) (width 0.2) (layer "F.Cu") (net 6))
 (segment (start 137.122 104.464) (end 138.5 103.086) (width 0.2) (layer "F.Cu") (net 6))
 (segment (start 135 103.952) (end 134.988 103.939) (width 0.2) (layer "F.Cu") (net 6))
 (segment (start 132.45 95.05) (end 132.45 94.4517) (width 0.2) (layer "F.Cu") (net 6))
 (segment (start 134.988 103.939) (end 134.988 103.5125) (width 0.2) (layer "F.Cu") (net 6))
 (segment (start 134.988 103.5125) (end 134.988 103.512) (width 0.2) (layer "F.Cu") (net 6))
 (segment (start 137.5 101.5) (end 139.88 101.5) (width 0.2) (layer "F.Cu") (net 6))
 (segment (start 142 100.6252) (end 142 99.5) (width 0.2) (layer "F.Cu") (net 6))
 (segment (start 143.5 99.325) (end 142.325 99.325) (width 0.2) (layer "F.Cu") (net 6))
 (segment (start 135 104.025) (end 135 103.952) (width 0.2) (layer "F.Cu") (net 6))
 (segment (start 142 99.5) (end 142 99) (width 0.2) (layer "F.Cu") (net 6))
 (segment (start 142 101) (end 142 100.6252) (width 0.2) (layer "F.Cu") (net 6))
 (segment (start 142 99) (end 141.713 98.7125) (width 0.2) (layer "F.Cu") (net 6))
 (segment (start 133.5 100.275) (end 135.5 100.275) (width 0.2) (layer "F.Cu") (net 6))
 (segment (start 132.5 96.8483) (end 132.5 95) (width 0.2) (layer "F.Cu") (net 6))
 (segment (start 131.8483 97.5) (end 131.8483 100.99) (width 0.2) (layer "F.Cu") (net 6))
 (segment (start 132.4 95.1) (end 132.45 95.05) (width 0.2) (layer "F.Cu") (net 6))
 (segment (start 135.5 104.025) (end 135.5 104.245) (width 0.2) (layer "F.Cu") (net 6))
 (segment (start 134.9875 103.5125) (end 134.988 103.5125) (width 0.2) (layer "F.Cu") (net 6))
 (segment (start 143.5 99.325) (end 144.175 99.325) (width 0.2) (layer "F.Cu") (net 6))
 (segment (start 140.962 100.325) (end 140.9715 100.3155) (width 0.2) (layer "F.Cu") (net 10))
 (segment (start 140.9715 100.3155) (end 140.981 100.306) (width 0.2) (layer "F.Cu") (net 10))
 (segment (start 140.972 100.3155) (end 141 100.2875) (width 0.2) (layer "F.Cu") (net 10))
 (segment (start 140.9715 100.3155) (end 140.972 100.3155) (width 0.2) (layer "F.Cu") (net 10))
 (segment (start 139 100.325) (end 140.962 100.325) (width 0.2) (layer "F.Cu") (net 10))
 (segment (start 132.675 99.8789) (end 133.0539 99.5) (width 0.2) (layer "F.Cu") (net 3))
 (segment (start 139.793 99.0753) (end 139.793 98.2764) (width 0.2) (layer "F.Cu") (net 3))
 (segment (start 136.9011 97.9028) (end 135.5 96.5017) (width 0.2) (layer "F.Cu") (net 3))
 (segment (start 139.3683 99.5) (end 139.793 99.0753) (width 0.2) (layer "F.Cu") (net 3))
 (segment (start 135.5 102.5) (end 135.5 102.0608) (width 0.2) (layer "F.Cu") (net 3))
 (segment (start 139.4194 97.9028) (end 136.9011 97.9028) (width 0.2) (layer "F.Cu") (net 3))
 (segment (start 134.0638 102.0608) (end 132.675 100.672) (width 0.2) (layer "F.Cu") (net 3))
 (segment (start 133.0539 99.5) (end 139.3683 99.5) (width 0.2) (layer "F.Cu") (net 3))
 (segment (start 135.5 95) (end 135.5 96.5017) (width 0.2) (layer "F.Cu") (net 3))
 (segment (start 132.675 100.672) (end 132.675 99.8789) (width 0.2) (layer "F.Cu") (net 3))
 (segment (start 139.793 98.2764) (end 139.4194 97.9028) (width 0.2) (layer "F.Cu") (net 3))
 (segment (start 135.5 102.0608) (end 134.0638 102.0608) (width 0.2) (layer "F.Cu") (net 3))
 (segment (start 138.5 95) (end 138.5 96.5017) (width 0.2) (layer "F.Cu") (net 1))
 (segment (start 136.5 101.835) (end 136.5 102.5) (width 0.2) (layer "F.Cu") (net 1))
 (segment (start 138.5 96.5017) (end 137.777 96.5017) (width 0.2) (layer "F.Cu") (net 1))
 (segment (start 137.777 96.5017) (end 137.1504 97.1283) (width 0.2) (layer "F.Cu") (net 1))
 (via (at 137.1504 97.1283) (size 0.6) (drill 0.3) (layers "F.Cu" "B.Cu") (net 1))
 (via (at 136.5 101.835) (size 0.6) (drill 0.3) (layers "F.Cu" "B.Cu") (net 1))
 (segment (start 136.5 97.7787) (end 137.1504 97.1283) (width 0.2) (layer "B.Cu") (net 1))
 (segment (start 136.5 101.835) (end 136.5 97.7787) (width 0.2) (layer "B.Cu") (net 1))
 (segment (start 135 102.5) (end 133.9329 102.5) (width 0.2) (layer "F.Cu") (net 4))
 (segment (start 132.2733 100.8404) (end 132.2733 98.2288) (width 0.2) (layer "F.Cu") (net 4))
 (segment (start 133.9329 102.5) (end 132.2733 100.8404) (width 0.2) (layer "F.Cu") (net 4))
 (segment (start 133.4599 93.4983) (end 137 93.4983) (width 0.2) (layer "F.Cu") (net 4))
 (segment (start 133.2983 97.2038) (end 133.2983 93.6599) (width 0.2) (layer "F.Cu") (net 4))
 (segment (start 137 95) (end 137 93.4983) (width 0.2) (layer "F.Cu") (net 4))
 (segment (start 133.2983 93.6599) (end 133.4599 93.4983) (width 0.2) (layer "F.Cu") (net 4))
 (segment (start 132.2733 98.2288) (end 133.2983 97.2038) (width 0.2) (layer "F.Cu") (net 4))
 (segment (start 140 96.5017) (end 139.2006 97.3011) (width 0.2) (layer "F.Cu") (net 2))
 (segment (start 136 102.9392) (end 136 103.0056) (width 0.2) (layer "F.Cu") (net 2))
 (segment (start 143.5 97) (end 143.5 97.675) (width 0.2) (layer "F.Cu") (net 2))
 (segment (start 140 96.5017) (end 140.0017 96.5) (width 0.2) (layer "F.Cu") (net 2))
 (segment (start 136 103.0056) (end 135.8404 103.1652) (width 0.2) (layer "F.Cu") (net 2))
 (segment (start 143 96.5) (end 143.5 97) (width 0.2) (layer "F.Cu") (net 2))
 (segment (start 140 95) (end 140 96.5017) (width 0.2) (layer "F.Cu") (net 2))
 (segment (start 139.2006 97.3011) (end 137.973 97.3011) (width 0.2) (layer "F.Cu") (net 2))
 (segment (start 140.0017 96.5) (end 143 96.5) (width 0.2) (layer "F.Cu") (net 2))
 (segment (start 136 102.5) (end 136 102.9392) (width 0.2) (layer "F.Cu") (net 2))
 (via (at 135.8404 103.1652) (size 0.6) (drill 0.3) (layers "F.Cu" "B.Cu") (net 2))
 (via (at 137.973 97.3011) (size 0.6) (drill 0.3) (layers "F.Cu" "B.Cu") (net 2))
 (segment (start 137.1312 99.0441) (end 137.1312 102.633271) (width 0.2) (layer "B.Cu") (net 2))
 (segment (start 137.013 103) (end 136.8478 103.1652) (width 0.2) (layer "B.Cu") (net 2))
 (segment (start 137.973 97.3011) (end 136.9565 98.3176) (width 0.2) (layer "B.Cu") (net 2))
 (segment (start 136.9565 98.8694) (end 137.1312 99.0441) (width 0.2) (layer "B.Cu") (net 2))
 (segment (start 136.8478 103.1652) (end 135.8404 103.1652) (width 0.2) (layer "B.Cu") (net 2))
 (segment (start 136.9565 98.3176) (end 136.9565 98.8694) (width 0.2) (layer "B.Cu") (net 2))
 (segment (start 137.013 102.751471) (end 137.013 103) (width 0.2) (layer "B.Cu") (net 2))
 (segment (start 137.1312 102.633271) (end 137.013 102.751471) (width 0.2) (layer "B.Cu") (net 2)))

